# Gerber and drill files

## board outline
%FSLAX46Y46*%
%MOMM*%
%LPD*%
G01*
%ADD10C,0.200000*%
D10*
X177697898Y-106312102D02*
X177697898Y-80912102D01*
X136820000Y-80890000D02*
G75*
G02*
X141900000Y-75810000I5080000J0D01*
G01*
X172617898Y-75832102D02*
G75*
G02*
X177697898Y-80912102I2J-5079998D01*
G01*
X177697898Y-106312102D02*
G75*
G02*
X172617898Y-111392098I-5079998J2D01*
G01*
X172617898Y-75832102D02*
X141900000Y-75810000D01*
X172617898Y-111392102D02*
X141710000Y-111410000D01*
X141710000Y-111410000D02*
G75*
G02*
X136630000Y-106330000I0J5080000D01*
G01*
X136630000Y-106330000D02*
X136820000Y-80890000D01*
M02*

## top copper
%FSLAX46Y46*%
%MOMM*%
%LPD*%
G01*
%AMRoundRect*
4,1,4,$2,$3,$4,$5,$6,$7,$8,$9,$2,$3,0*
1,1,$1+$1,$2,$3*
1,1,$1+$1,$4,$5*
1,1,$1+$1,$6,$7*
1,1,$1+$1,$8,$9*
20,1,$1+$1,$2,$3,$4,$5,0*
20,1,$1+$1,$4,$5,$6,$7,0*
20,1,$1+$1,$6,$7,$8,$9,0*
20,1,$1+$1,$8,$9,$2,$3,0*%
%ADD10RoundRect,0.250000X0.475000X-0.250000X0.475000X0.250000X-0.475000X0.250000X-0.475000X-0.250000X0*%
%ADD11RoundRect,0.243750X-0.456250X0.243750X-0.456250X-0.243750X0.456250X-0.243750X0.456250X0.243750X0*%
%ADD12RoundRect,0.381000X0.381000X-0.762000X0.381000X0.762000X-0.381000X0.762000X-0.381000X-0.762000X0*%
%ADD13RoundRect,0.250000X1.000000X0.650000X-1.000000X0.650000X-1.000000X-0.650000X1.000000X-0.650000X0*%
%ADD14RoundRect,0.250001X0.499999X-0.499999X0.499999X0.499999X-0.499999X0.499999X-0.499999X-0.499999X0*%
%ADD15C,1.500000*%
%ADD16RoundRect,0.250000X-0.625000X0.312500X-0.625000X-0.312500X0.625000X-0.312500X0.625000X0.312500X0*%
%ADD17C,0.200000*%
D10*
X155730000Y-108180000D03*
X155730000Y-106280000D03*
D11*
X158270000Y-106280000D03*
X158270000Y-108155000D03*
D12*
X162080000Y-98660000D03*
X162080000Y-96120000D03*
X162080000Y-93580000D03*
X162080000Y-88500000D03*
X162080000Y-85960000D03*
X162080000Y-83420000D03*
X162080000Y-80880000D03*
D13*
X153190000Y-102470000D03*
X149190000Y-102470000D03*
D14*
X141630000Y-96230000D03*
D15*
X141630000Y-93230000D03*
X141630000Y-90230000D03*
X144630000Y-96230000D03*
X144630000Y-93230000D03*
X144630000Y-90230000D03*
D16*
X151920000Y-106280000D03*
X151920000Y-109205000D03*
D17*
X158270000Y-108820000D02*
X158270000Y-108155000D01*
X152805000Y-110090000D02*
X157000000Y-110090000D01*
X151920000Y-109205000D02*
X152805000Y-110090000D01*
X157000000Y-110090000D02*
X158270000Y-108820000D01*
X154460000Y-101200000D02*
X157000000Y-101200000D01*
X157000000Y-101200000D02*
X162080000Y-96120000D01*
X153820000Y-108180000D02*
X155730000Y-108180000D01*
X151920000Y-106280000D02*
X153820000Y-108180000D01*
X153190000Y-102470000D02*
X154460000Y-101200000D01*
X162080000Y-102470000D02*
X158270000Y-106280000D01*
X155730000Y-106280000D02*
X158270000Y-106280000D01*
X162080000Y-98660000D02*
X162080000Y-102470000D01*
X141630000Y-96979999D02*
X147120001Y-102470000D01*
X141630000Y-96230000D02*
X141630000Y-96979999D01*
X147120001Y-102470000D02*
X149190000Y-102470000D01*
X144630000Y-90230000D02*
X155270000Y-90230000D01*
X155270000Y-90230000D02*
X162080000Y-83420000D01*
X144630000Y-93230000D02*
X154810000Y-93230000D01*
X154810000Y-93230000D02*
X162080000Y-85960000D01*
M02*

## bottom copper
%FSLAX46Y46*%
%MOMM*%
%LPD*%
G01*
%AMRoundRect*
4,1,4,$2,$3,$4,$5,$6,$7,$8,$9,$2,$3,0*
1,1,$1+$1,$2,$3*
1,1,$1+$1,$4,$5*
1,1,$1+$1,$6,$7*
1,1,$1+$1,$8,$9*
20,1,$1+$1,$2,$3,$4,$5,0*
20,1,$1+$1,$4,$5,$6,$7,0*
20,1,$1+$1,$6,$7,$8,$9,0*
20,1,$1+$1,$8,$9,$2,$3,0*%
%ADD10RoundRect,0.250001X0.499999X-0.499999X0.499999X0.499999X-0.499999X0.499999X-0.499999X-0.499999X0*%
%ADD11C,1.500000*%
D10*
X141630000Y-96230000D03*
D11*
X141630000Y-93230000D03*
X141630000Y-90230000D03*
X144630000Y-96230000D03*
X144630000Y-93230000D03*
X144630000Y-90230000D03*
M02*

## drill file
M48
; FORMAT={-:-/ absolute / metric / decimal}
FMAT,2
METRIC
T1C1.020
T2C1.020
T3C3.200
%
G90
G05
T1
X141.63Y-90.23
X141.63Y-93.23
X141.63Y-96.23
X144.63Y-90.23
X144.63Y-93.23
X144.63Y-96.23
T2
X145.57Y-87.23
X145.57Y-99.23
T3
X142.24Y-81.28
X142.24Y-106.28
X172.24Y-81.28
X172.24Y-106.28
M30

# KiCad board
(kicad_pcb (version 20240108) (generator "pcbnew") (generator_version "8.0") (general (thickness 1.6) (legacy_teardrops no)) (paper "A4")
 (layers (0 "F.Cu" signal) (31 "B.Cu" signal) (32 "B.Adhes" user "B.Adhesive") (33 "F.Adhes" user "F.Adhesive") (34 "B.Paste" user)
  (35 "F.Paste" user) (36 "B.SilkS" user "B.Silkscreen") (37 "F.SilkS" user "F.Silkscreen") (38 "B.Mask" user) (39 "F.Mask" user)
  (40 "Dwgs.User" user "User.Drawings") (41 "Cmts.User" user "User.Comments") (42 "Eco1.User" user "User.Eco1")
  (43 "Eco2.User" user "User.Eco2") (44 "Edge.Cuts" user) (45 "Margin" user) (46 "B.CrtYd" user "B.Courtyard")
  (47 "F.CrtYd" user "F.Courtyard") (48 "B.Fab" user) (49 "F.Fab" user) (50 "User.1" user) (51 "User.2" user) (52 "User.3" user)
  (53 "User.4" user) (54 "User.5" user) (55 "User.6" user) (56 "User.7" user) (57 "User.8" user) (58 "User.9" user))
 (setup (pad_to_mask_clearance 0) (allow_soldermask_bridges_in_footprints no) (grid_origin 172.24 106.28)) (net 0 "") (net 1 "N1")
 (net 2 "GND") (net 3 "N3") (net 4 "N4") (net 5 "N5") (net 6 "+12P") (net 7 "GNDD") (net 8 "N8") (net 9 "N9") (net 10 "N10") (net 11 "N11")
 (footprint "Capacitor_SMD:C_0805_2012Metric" (layer "F.Cu") (at 155.73 107.23 90)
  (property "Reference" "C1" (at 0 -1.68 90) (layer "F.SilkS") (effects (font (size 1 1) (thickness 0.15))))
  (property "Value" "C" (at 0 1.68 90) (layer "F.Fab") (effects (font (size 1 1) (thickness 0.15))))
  (pad "1" smd roundrect (at -0.95 0 90) (size 1 1.45) (layers "F.Cu" "F.Paste" "F.Mask") (roundrect_rratio 0.25) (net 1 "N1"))
  (pad "2" smd roundrect (at 0.95 0 90) (size 1 1.45) (layers "F.Cu" "F.Paste" "F.Mask") (roundrect_rratio 0.25) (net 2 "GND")))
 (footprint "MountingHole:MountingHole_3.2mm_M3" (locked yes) (layer "F.Cu") (at 142.24 81.28)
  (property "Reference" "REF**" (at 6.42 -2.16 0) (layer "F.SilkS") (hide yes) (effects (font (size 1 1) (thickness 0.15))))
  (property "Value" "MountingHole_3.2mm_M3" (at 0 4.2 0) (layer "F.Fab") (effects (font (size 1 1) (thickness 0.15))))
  (pad "" np_thru_hole circle (at 0 0) (size 3.2 3.2) (drill 3.2) (layers "F&B.Cu" "*.Mask")))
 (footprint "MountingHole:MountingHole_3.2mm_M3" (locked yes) (layer "F.Cu") (at 172.24 106.28)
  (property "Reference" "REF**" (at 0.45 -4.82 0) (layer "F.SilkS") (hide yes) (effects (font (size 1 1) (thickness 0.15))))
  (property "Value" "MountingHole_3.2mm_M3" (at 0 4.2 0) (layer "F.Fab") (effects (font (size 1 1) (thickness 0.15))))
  (pad "" np_thru_hole circle (at 0 0) (size 3.2 3.2) (drill 3.2) (layers "F&B.Cu" "*.Mask")))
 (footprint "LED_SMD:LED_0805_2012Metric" (layer "F.Cu") (at 158.27 107.2175 -90)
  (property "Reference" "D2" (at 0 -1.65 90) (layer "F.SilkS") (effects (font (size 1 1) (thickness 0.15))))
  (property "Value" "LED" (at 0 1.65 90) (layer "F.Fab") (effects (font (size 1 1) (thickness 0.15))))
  (pad "1" smd roundrect (at -0.9375 0 270) (size 0.975 1.4) (layers "F.Cu" "F.Paste" "F.Mask") (roundrect_rratio 0.25) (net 2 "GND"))
  (pad "2" smd roundrect (at 0.9375 0 270) (size 0.975 1.4) (layers "F.Cu" "F.Paste" "F.Mask") (roundrect_rratio 0.25) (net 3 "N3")))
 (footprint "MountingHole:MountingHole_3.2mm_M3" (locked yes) (layer "F.Cu") (at 142.24 106.28)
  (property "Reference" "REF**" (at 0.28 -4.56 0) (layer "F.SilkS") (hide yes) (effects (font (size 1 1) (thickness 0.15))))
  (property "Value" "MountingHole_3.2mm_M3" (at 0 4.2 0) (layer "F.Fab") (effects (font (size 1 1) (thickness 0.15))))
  (pad "" np_thru_hole circle (at 0 0) (size 3.2 3.2) (drill 3.2) (layers "F&B.Cu" "*.Mask")))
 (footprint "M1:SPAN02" (layer "F.Cu") (at 162.08 98.66 90)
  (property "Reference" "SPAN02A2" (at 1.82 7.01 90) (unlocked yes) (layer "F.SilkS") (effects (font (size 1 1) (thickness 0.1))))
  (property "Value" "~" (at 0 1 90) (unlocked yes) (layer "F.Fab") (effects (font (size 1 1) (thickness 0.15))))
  (pad "1" smd roundrect (at 0 0 90) (size 2.286 1.524) (layers "F.Cu" "F.Paste" "F.Mask") (roundrect_rratio 0.25) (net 2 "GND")
   (thermal_bridge_angle 45))
  (pad "2" smd roundrect (at 2.54 0 90) (size 2.286 1.524) (layers "F.Cu" "F.Paste" "F.Mask") (roundrect_rratio 0.25) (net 1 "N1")
   (thermal_bridge_angle 45))
  (pad "3" smd roundrect (at 5.08 0 90) (size 2.286 1.524) (layers "F.Cu" "F.Paste" "F.Mask") (roundrect_rratio 0.25) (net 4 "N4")
   (thermal_bridge_angle 45))
  (pad "5" smd roundrect (at 10.16 0 90) (size 2.286 1.524) (layers "F.Cu" "F.Paste" "F.Mask") (roundrect_rratio 0.25) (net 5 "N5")
   (thermal_bridge_angle 45))
  (pad "6" smd roundrect (at 12.7 0 90) (size 2.286 1.524) (layers "F.Cu" "F.Paste" "F.Mask") (roundrect_rratio 0.25) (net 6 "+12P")
   (thermal_bridge_angle 45))
  (pad "7" smd roundrect (at 15.24 0 90) (size 2.286 1.524) (layers "F.Cu" "F.Paste" "F.Mask") (roundrect_rratio 0.25) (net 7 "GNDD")
   (thermal_bridge_angle 45))
  (pad "8" smd roundrect (at 17.78 0 90) (size 2.286 1.524) (layers "F.Cu" "F.Paste" "F.Mask") (roundrect_rratio 0.25) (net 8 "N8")
   (thermal_bridge_angle 45)))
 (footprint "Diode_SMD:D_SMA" (layer "F.Cu") (at 151.19 102.47 180)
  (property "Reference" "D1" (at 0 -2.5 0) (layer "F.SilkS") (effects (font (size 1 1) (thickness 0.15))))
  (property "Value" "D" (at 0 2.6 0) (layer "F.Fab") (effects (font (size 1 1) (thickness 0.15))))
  (pad "1" smd roundrect (at -2 0 180) (size 2.5 1.8) (layers "F.Cu" "F.Paste" "F.Mask") (roundrect_rratio 0.1388888889) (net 1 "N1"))
  (pad "2" smd roundrect (at 2 0 180) (size 2.5 1.8) (layers "F.Cu" "F.Paste" "F.Mask") (roundrect_rratio 0.1388888889) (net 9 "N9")))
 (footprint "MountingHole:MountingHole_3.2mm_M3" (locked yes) (layer "F.Cu") (at 172.24 81.28)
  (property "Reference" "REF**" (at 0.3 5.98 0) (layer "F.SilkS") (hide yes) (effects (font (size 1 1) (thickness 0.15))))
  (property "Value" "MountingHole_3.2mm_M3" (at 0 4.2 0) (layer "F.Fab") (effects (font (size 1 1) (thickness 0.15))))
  (pad "" np_thru_hole circle (at 0 0) (size 3.2 3.2) (drill 3.2) (layers "F&B.Cu" "*.Mask")))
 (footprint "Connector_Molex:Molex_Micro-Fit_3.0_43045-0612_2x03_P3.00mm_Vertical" (layer "F.Cu") (at 141.63 96.23 90)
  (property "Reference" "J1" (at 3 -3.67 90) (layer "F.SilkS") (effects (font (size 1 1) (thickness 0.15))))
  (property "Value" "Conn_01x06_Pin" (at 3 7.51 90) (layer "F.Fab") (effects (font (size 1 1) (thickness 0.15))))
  (pad "" np_thru_hole circle (at -3 3.94 90) (size 1.02 1.02) (drill 1.02) (layers "*.Cu" "*.Mask"))
  (pad "" np_thru_hole circle (at 9 3.94 90) (size 1.02 1.02) (drill 1.02) (layers "*.Cu" "*.Mask"))
  (pad "1" thru_hole roundrect (at 0 0 90) (size 1.5 1.5) (drill 1.02) (layers "*.Cu" "*.Mask") (remove_unused_layers no)
   (roundrect_rratio 0.166667) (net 9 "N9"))
  (pad "2" thru_hole circle (at 3 0 90) (size 1.5 1.5) (drill 1.02) (layers "*.Cu" "*.Mask") (remove_unused_layers no) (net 2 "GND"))
  (pad "3" thru_hole circle (at 6 0 90) (size 1.5 1.5) (drill 1.02) (layers "*.Cu" "*.Mask") (remove_unused_layers no) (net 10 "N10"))
  (pad "4" thru_hole circle (at 0 3 90) (size 1.5 1.5) (drill 1.02) (layers "*.Cu" "*.Mask") (remove_unused_layers no) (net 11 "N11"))
  (pad "5" thru_hole circle (at 3 3 90) (size 1.5 1.5) (drill 1.02) (layers "*.Cu" "*.Mask") (remove_unused_layers no) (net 6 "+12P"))
  (pad "6" thru_hole circle (at 6 3 90) (size 1.5 1.5) (drill 1.02) (layers "*.Cu" "*.Mask") (remove_unused_layers no) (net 7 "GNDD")))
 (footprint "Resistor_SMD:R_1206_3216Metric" (layer "F.Cu") (at 151.92 107.7425 -90)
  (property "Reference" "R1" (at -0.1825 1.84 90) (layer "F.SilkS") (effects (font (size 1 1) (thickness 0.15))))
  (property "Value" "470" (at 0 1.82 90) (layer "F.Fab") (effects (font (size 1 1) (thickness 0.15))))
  (pad "1" smd roundrect (at -1.4625 0 270) (size 1.125 1.75) (layers "F.Cu" "F.Paste" "F.Mask") (roundrect_rratio 0.222222) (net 1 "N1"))
  (pad "2" smd roundrect (at 1.4625 0 270) (size 1.125 1.75) (layers "F.Cu" "F.Paste" "F.Mask") (roundrect_rratio 0.222222) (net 3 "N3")))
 (gr_line (start 177.697898 106.312102) (end 177.697898 80.912102) (stroke (width 0.2) (type default)) (layer "Edge.Cuts"))
 (gr_arc (start 136.82 80.89) (mid 138.307898 77.297898) (end 141.9 75.81) (stroke (width 0.2) (type default)) (layer "Edge.Cuts"))
 (gr_arc (start 172.617898 75.832102) (mid 176.21 77.32) (end 177.697898 80.912102) (stroke (width 0.2) (type default)) (layer "Edge.Cuts"))
 (gr_arc (start 177.697898 106.312102) (mid 176.21 109.904204) (end 172.617898 111.392102) (stroke (width 0.2) (type default))
  (layer "Edge.Cuts"))
 (gr_line (start 172.617898 75.832102) (end 141.9 75.81) (stroke (width 0.2) (type default)) (layer "Edge.Cuts"))
 (gr_line (start 172.617898 111.392102) (end 141.71 111.41) (stroke (width 0.2) (type default)) (layer "Edge.Cuts"))
 (gr_arc (start 141.71 111.41) (mid 138.117898 109.922102) (end 136.63 106.33) (stroke (width 0.2) (type default)) (layer "Edge.Cuts"))
 (gr_line (start 136.63 106.33) (end 136.82 80.89) (stroke (width 0.2) (type default)) (layer "Edge.Cuts"))
 (segment (start 158.27 108.82) (end 158.27 108.155) (width 0.2) (layer "F.Cu") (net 3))
 (segment (start 152.805 110.09) (end 157 110.09) (width 0.2) (layer "F.Cu") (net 3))
 (segment (start 151.92 109.205) (end 152.805 110.09) (width 0.2) (layer "F.Cu") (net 3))
 (segment (start 157 110.09) (end 158.27 108.82) (width 0.2) (layer "F.Cu") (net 3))
 (segment (start 154.46 101.2) (end 157 101.2) (width 0.2) (layer "F.Cu") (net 1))
 (segment (start 157 101.2) (end 162.08 96.12) (width 0.2) (layer "F.Cu") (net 1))
 (segment (start 153.82 108.18) (end 155.73 108.18) (width 0.2) (layer "F.Cu") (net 1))
 (segment (start 151.92 106.28) (end 153.82 108.18) (width 0.2) (layer "F.Cu") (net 1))
 (segment (start 153.19 102.47) (end 154.46 101.2) (width 0.2) (layer "F.Cu") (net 1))
 (segment (start 162.08 102.47) (end 158.27 106.28) (width 0.2) (layer "F.Cu") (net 2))
 (segment (start 155.73 106.28) (end 158.27 106.28) (width 0.2) (layer "F.Cu") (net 2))
 (segment (start 162.08 98.66) (end 162.08 102.47) (width 0.2) (layer "F.Cu") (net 2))
 (segment (start 141.63 96.979999) (end 147.120001 102.47) (width 0.2) (layer "F.Cu") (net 9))
 (segment (start 141.63 96.23) (end 141.63 96.979999) (width 0.2) (layer "F.Cu") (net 9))
 (segment (start 147.120001 102.47) (end 149.19 102.47) (width 0.2) (layer "F.Cu") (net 9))
 (segment (start 144.63 90.23) (end 155.27 90.23) (width 0.2) (layer "F.Cu") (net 7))
 (segment (start 155.27 90.23) (end 162.08 83.42) (width 0.2) (layer "F.Cu") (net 7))
 (segment (start 144.63 93.23) (end 154.81 93.23) (width 0.2) (layer "F.Cu") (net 6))
 (segment (start 154.81 93.23) (end 162.08 85.96) (width 0.2) (layer "F.Cu") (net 6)))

